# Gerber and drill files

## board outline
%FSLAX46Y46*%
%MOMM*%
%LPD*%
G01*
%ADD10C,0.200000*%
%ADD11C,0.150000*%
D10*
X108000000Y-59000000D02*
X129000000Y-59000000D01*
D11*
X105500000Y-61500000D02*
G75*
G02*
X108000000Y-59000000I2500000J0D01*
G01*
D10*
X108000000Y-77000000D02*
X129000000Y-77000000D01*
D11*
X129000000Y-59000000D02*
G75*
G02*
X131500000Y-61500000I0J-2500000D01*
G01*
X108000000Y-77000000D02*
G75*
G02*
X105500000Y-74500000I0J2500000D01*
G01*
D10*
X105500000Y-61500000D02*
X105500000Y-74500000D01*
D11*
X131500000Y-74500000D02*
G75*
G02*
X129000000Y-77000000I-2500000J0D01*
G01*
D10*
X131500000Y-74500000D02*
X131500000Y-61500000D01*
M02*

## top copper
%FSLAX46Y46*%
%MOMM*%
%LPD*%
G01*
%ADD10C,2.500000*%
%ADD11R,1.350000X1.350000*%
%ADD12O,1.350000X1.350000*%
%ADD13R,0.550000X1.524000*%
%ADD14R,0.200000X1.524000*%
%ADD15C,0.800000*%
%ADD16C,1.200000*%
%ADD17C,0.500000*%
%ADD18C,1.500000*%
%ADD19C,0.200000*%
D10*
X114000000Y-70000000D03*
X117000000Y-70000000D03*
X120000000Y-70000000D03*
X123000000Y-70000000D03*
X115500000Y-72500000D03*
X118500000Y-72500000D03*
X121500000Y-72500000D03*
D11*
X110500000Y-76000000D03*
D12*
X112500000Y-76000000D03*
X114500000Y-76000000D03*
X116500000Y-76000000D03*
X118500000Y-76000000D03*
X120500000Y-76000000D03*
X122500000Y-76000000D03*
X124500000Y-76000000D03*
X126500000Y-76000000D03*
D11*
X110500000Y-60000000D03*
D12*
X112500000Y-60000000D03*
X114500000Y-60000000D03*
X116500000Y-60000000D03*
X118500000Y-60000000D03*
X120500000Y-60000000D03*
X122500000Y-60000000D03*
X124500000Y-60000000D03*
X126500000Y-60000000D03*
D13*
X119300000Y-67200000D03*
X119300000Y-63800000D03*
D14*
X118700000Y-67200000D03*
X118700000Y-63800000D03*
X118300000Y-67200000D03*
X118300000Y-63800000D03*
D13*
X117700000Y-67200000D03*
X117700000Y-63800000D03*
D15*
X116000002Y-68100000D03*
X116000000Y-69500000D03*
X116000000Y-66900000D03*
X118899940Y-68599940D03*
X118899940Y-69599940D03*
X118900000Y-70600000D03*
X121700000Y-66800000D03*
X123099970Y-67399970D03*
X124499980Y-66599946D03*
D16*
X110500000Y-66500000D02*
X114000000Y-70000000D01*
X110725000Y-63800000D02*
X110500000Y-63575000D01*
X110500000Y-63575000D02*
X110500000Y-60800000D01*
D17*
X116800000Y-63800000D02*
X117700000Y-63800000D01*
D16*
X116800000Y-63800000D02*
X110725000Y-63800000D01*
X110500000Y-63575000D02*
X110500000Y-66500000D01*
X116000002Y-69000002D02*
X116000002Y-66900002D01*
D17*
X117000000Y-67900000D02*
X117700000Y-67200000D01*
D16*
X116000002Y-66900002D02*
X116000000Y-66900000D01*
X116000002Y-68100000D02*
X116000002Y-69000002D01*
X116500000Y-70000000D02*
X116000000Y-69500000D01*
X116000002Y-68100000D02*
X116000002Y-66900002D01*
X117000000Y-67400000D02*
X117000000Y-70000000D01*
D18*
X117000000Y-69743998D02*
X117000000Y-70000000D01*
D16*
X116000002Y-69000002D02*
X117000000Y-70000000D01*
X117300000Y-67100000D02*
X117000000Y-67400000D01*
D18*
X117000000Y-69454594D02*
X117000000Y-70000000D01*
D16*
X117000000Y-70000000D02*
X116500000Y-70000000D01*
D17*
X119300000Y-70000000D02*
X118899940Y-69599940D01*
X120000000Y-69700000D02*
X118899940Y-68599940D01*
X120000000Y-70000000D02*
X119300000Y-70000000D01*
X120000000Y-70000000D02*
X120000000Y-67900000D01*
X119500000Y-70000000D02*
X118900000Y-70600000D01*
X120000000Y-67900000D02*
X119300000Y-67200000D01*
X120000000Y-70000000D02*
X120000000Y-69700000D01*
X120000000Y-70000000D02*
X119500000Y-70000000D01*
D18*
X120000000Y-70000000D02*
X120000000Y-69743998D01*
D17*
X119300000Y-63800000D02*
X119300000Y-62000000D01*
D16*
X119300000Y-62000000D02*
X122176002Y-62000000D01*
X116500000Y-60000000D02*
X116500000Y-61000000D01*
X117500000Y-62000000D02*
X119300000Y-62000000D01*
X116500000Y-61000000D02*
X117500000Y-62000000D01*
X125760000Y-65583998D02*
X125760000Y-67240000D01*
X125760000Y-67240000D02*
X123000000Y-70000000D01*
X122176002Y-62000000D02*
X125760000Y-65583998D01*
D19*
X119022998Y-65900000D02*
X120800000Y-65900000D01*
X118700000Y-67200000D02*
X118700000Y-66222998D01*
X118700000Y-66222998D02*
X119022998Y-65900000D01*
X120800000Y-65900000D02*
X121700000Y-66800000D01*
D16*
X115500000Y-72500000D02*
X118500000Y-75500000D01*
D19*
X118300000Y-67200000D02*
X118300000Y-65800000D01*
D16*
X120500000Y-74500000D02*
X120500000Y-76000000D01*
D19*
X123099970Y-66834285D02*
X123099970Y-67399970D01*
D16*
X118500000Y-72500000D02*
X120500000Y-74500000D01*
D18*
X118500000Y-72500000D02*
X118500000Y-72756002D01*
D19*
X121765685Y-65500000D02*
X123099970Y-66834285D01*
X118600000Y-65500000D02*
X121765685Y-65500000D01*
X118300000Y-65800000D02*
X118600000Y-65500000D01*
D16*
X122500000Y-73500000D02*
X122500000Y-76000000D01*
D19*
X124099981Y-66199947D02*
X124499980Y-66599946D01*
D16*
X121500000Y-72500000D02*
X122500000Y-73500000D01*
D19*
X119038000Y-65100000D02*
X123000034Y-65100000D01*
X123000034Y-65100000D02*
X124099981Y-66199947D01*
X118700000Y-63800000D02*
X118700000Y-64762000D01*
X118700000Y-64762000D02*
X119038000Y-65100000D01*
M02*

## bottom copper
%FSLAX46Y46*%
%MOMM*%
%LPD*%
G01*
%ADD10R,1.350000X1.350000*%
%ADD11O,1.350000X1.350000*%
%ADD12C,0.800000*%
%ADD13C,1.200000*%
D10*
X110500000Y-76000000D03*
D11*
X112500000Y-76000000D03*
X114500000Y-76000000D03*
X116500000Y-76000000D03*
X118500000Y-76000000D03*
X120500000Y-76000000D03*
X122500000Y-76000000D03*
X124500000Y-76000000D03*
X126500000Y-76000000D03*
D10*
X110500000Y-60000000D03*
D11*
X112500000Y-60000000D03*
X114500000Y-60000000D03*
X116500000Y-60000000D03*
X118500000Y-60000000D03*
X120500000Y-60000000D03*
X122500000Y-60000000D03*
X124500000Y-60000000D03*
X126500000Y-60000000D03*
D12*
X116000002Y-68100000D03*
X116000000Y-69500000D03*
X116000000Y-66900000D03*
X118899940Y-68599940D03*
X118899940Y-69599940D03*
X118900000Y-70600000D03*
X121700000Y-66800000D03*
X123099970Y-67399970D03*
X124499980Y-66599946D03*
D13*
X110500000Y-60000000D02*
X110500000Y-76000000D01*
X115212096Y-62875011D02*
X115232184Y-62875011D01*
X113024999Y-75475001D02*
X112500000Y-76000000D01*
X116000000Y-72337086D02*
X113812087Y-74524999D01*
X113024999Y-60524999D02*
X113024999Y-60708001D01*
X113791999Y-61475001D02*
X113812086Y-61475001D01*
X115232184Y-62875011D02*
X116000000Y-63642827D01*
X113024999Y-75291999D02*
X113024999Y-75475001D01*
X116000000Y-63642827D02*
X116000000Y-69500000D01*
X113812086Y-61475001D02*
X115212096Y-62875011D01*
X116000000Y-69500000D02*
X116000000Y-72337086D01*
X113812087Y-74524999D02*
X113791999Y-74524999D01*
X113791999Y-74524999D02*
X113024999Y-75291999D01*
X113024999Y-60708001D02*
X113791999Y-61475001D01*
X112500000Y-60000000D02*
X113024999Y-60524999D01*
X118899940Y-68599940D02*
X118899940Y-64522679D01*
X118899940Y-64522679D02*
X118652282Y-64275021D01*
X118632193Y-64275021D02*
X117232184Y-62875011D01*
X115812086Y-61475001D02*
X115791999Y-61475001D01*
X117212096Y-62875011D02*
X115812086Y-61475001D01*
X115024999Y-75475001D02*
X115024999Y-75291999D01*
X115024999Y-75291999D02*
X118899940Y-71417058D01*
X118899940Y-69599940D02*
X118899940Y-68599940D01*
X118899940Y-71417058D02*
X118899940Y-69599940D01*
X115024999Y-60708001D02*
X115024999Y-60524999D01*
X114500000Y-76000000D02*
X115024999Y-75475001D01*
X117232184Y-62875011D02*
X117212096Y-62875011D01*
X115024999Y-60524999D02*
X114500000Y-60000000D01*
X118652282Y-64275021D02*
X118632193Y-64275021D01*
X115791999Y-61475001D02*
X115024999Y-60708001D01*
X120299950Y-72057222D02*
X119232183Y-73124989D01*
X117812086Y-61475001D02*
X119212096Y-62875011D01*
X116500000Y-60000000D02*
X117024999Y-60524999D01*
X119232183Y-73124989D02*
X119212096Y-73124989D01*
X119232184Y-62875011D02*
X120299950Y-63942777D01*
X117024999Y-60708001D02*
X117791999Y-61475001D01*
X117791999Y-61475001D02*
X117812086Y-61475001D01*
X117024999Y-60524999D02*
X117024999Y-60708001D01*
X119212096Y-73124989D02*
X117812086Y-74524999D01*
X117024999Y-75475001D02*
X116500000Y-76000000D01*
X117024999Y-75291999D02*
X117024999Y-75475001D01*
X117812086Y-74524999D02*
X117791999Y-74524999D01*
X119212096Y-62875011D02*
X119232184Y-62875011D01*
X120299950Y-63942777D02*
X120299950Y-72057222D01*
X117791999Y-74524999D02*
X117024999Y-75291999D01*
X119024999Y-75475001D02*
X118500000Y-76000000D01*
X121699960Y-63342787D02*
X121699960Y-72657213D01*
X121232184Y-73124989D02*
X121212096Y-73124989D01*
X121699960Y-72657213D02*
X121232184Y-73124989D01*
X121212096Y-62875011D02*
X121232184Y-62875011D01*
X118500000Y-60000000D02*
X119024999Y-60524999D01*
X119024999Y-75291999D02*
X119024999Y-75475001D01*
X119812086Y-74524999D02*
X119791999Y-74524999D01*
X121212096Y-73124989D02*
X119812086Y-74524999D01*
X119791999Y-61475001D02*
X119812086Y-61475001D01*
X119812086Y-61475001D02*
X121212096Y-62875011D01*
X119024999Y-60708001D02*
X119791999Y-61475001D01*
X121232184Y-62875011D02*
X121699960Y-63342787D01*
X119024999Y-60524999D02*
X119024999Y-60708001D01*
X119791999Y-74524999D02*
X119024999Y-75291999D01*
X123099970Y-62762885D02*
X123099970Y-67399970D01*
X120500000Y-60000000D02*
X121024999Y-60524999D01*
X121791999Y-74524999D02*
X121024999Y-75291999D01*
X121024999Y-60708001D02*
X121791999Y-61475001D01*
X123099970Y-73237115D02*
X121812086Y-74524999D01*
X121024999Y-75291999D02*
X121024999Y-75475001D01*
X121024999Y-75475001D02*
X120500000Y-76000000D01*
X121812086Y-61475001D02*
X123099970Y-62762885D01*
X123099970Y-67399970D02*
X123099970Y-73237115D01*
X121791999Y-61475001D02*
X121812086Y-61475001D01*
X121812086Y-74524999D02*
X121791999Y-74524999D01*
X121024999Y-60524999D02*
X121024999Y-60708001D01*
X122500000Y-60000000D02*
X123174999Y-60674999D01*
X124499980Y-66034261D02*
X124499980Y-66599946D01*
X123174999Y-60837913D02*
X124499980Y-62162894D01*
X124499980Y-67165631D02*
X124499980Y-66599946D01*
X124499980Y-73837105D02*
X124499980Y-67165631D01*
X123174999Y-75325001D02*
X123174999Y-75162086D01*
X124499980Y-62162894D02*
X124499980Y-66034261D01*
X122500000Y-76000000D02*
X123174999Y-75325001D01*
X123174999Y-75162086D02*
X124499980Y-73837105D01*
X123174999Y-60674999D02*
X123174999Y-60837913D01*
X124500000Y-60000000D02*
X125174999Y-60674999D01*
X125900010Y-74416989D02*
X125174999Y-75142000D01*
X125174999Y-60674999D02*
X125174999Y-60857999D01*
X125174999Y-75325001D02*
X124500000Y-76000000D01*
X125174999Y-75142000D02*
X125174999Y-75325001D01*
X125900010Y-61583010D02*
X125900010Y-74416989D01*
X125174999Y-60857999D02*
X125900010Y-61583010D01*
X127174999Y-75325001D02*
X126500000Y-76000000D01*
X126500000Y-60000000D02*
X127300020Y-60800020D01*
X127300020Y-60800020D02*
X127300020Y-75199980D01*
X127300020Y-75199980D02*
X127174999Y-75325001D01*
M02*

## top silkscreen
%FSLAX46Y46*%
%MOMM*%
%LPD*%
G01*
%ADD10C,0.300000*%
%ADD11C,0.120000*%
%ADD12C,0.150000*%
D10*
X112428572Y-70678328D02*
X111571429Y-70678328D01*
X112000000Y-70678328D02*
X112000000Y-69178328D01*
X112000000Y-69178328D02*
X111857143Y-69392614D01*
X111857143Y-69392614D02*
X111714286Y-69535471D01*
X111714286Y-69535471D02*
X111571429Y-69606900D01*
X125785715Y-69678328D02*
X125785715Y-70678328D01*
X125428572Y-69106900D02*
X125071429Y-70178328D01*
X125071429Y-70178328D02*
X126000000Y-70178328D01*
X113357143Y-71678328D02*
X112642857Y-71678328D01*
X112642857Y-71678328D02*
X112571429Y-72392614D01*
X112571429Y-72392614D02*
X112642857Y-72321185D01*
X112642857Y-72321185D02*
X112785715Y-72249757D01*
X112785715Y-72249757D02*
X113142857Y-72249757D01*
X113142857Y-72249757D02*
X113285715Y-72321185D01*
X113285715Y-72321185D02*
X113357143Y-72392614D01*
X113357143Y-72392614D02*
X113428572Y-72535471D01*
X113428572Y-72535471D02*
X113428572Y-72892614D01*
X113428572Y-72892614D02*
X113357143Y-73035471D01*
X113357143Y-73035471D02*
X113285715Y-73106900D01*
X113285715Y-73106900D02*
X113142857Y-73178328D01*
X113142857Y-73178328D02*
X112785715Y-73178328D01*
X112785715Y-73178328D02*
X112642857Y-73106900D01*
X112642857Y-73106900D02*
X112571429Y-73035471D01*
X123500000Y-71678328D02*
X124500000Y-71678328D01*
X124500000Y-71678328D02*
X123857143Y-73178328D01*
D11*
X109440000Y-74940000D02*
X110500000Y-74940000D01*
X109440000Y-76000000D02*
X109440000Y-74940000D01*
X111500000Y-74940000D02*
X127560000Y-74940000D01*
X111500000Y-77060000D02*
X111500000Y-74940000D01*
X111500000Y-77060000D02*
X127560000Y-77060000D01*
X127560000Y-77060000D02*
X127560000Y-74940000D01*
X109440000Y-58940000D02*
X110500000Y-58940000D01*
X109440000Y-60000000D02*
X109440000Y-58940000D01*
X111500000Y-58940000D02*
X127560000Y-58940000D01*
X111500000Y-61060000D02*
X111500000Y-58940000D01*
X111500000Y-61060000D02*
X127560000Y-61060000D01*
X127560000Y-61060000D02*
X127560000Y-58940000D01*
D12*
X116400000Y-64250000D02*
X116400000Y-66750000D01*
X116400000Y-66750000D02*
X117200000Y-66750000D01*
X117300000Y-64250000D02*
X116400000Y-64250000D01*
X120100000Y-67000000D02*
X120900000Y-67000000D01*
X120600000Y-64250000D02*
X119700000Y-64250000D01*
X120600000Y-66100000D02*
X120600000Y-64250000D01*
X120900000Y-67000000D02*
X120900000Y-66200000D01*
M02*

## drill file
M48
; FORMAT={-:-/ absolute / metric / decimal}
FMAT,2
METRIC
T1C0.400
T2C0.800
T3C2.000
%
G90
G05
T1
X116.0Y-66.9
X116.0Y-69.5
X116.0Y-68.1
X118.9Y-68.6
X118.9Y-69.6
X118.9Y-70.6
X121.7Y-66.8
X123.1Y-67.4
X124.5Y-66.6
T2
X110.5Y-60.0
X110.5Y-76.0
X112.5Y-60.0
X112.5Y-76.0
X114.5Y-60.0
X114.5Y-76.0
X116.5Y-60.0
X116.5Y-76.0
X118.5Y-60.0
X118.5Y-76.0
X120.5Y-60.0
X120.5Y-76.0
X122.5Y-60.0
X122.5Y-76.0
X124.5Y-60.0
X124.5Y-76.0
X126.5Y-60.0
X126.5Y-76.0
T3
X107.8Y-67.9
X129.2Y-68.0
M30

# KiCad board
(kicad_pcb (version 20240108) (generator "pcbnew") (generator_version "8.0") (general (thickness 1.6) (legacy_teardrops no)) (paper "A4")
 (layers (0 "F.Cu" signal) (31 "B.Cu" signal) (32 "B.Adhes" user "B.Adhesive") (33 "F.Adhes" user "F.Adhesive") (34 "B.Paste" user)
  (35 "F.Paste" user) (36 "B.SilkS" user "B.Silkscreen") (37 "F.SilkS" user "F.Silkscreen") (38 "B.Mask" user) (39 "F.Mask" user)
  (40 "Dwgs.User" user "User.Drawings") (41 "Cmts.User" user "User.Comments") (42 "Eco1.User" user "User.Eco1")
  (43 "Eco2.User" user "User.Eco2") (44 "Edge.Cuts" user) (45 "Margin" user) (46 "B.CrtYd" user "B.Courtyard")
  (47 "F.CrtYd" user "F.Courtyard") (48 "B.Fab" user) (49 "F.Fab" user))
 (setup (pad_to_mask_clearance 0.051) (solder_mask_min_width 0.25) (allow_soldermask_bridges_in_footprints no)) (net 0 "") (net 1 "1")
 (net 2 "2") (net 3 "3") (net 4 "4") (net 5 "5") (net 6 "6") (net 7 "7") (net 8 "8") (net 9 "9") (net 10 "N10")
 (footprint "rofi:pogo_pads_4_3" (layer "F.Cu") (at 118.5 70)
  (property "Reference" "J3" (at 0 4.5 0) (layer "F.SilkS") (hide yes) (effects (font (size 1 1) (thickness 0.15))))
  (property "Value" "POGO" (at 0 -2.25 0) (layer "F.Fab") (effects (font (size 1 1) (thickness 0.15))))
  (pad "1" smd circle (at -4.5 0) (size 2.5 2.5) (layers "F.Cu" "F.Paste" "F.Mask") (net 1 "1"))
  (pad "2" smd circle (at -1.5 0) (size 2.5 2.5) (layers "F.Cu" "F.Paste" "F.Mask") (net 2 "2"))
  (pad "3" smd circle (at 1.5 0) (size 2.5 2.5) (layers "F.Cu" "F.Paste" "F.Mask") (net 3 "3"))
  (pad "4" smd circle (at 4.5 0) (size 2.5 2.5) (layers "F.Cu" "F.Paste" "F.Mask") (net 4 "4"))
  (pad "5" smd circle (at -3 2.5) (size 2.5 2.5) (layers "F.Cu" "F.Paste" "F.Mask") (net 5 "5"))
  (pad "6" smd circle (at 0 2.5) (size 2.5 2.5) (layers "F.Cu" "F.Paste" "F.Mask") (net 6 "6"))
  (pad "7" smd circle (at 3 2.5) (size 2.5 2.5) (layers "F.Cu" "F.Paste" "F.Mask") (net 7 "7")))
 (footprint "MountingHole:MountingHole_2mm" (layer "F.Cu") (at 129.2 68)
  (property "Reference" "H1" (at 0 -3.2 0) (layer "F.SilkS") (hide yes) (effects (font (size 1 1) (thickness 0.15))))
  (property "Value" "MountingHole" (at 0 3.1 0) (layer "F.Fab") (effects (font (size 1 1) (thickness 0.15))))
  (pad "" np_thru_hole circle (at 0 0) (size 2 2) (drill 2) (layers "*.Cu" "*.Mask")))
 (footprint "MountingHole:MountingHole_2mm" (layer "F.Cu") (at 107.8 67.9)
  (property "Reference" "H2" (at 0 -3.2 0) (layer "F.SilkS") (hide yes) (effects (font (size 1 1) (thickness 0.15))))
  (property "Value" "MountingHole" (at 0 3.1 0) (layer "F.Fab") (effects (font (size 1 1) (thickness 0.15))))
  (pad "" np_thru_hole circle (at 0 0) (size 2 2) (drill 2) (layers "*.Cu" "*.Mask")))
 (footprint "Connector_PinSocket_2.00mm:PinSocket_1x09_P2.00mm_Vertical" (layer "F.Cu") (at 110.5 76 90)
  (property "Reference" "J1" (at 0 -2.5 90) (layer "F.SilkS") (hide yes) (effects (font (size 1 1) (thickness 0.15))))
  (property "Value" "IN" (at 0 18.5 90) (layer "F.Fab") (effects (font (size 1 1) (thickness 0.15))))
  (fp_line (start 1.06 -1.06) (end 1.06 0) (stroke (width 0.12) (type solid)) (layer "F.SilkS"))
  (fp_line (start 0 -1.06) (end 1.06 -1.06) (stroke (width 0.12) (type solid)) (layer "F.SilkS"))
  (fp_line (start 1.06 1) (end 1.06 17.06) (stroke (width 0.12) (type solid)) (layer "F.SilkS"))
  (fp_line (start -1.06 1) (end 1.06 1) (stroke (width 0.12) (type solid)) (layer "F.SilkS"))
  (fp_line (start -1.06 1) (end -1.06 17.06) (stroke (width 0.12) (type solid)) (layer "F.SilkS"))
  (fp_line (start -1.06 17.06) (end 1.06 17.06) (stroke (width 0.12) (type solid)) (layer "F.SilkS"))
  (pad "1" thru_hole rect (at 0 0 90) (size 1.35 1.35) (drill 0.8) (layers "*.Cu" "*.Mask") (remove_unused_layers no) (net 1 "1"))
  (pad "2" thru_hole oval (at 0 2 90) (size 1.35 1.35) (drill 0.8) (layers "*.Cu" "*.Mask") (remove_unused_layers no) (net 2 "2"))
  (pad "3" thru_hole oval (at 0 4 90) (size 1.35 1.35) (drill 0.8) (layers "*.Cu" "*.Mask") (remove_unused_layers no) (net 3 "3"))
  (pad "4" thru_hole oval (at 0 6 90) (size 1.35 1.35) (drill 0.8) (layers "*.Cu" "*.Mask") (remove_unused_layers no) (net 4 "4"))
  (pad "5" thru_hole oval (at 0 8 90) (size 1.35 1.35) (drill 0.8) (layers "*.Cu" "*.Mask") (remove_unused_layers no) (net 5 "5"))
  (pad "6" thru_hole oval (at 0 10 90) (size 1.35 1.35) (drill 0.8) (layers "*.Cu" "*.Mask") (remove_unused_layers no) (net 6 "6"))
  (pad "7" thru_hole oval (at 0 12 90) (size 1.35 1.35) (drill 0.8) (layers "*.Cu" "*.Mask") (remove_unused_layers no) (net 7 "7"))
  (pad "8" thru_hole oval (at 0 14 90) (size 1.35 1.35) (drill 0.8) (layers "*.Cu" "*.Mask") (remove_unused_layers no) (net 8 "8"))
  (pad "9" thru_hole oval (at 0 16 90) (size 1.35 1.35) (drill 0.8) (layers "*.Cu" "*.Mask") (remove_unused_layers no) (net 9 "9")))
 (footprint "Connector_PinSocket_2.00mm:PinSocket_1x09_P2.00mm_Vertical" (layer "F.Cu") (at 110.5 60 90)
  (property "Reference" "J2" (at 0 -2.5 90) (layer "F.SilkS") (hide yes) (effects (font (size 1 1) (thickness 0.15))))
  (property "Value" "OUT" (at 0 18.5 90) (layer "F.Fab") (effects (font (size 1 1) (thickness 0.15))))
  (fp_line (start 1.06 -1.06) (end 1.06 0) (stroke (width 0.12) (type solid)) (layer "F.SilkS"))
  (fp_line (start 0 -1.06) (end 1.06 -1.06) (stroke (width 0.12) (type solid)) (layer "F.SilkS"))
  (fp_line (start 1.06 1) (end 1.06 17.06) (stroke (width 0.12) (type solid)) (layer "F.SilkS"))
  (fp_line (start -1.06 1) (end 1.06 1) (stroke (width 0.12) (type solid)) (layer "F.SilkS"))
  (fp_line (start -1.06 1) (end -1.06 17.06) (stroke (width 0.12) (type solid)) (layer "F.SilkS"))
  (fp_line (start -1.06 17.06) (end 1.06 17.06) (stroke (width 0.12) (type solid)) (layer "F.SilkS"))
  (pad "1" thru_hole rect (at 0 0 90) (size 1.35 1.35) (drill 0.8) (layers "*.Cu" "*.Mask") (remove_unused_layers no) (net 1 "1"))
  (pad "2" thru_hole oval (at 0 2 90) (size 1.35 1.35) (drill 0.8) (layers "*.Cu" "*.Mask") (remove_unused_layers no) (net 2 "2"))
  (pad "3" thru_hole oval (at 0 4 90) (size 1.35 1.35) (drill 0.8) (layers "*.Cu" "*.Mask") (remove_unused_layers no) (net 3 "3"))
  (pad "4" thru_hole oval (at 0 6 90) (size 1.35 1.35) (drill 0.8) (layers "*.Cu" "*.Mask") (remove_unused_layers no) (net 4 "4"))
  (pad "5" thru_hole oval (at 0 8 90) (size 1.35 1.35) (drill 0.8) (layers "*.Cu" "*.Mask") (remove_unused_layers no) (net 5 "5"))
  (pad "6" thru_hole oval (at 0 10 90) (size 1.35 1.35) (drill 0.8) (layers "*.Cu" "*.Mask") (remove_unused_layers no) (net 6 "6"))
  (pad "7" thru_hole oval (at 0 12 90) (size 1.35 1.35) (drill 0.8) (layers "*.Cu" "*.Mask") (remove_unused_layers no) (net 7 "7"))
  (pad "8" thru_hole oval (at 0 14 90) (size 1.35 1.35) (drill 0.8) (layers "*.Cu" "*.Mask") (remove_unused_layers no) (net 8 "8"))
  (pad "9" thru_hole oval (at 0 16 90) (size 1.35 1.35) (drill 0.8) (layers "*.Cu" "*.Mask") (remove_unused_layers no) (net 9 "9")))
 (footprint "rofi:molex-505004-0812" (layer "F.Cu") (at 118.5 65.5 180)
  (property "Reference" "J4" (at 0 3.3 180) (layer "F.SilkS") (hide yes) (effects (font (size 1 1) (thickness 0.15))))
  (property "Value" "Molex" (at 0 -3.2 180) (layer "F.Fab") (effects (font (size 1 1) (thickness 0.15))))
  (fp_line (start 2.1 1.25) (end 2.1 -1.25) (stroke (width 0.15) (type solid)) (layer "F.SilkS"))
  (fp_line (start 2.1 -1.25) (end 1.3 -1.25) (stroke (width 0.15) (type solid)) (layer "F.SilkS"))
  (fp_line (start 1.2 1.25) (end 2.1 1.25) (stroke (width 0.15) (type solid)) (layer "F.SilkS"))
  (fp_line (start -1.6 -1.5) (end -2.4 -1.5) (stroke (width 0.15) (type solid)) (layer "F.SilkS"))
  (fp_line (start -2.1 1.25) (end -1.2 1.25) (stroke (width 0.15) (type solid)) (layer "F.SilkS"))
  (fp_line (start -2.1 -0.6) (end -2.1 1.25) (stroke (width 0.15) (type solid)) (layer "F.SilkS"))
  (fp_line (start -2.4 -1.5) (end -2.4 -0.7) (stroke (width 0.15) (type solid)) (layer "F.SilkS"))
  (pad "1" smd rect (at -0.8 -1.7 180) (size 0.55 1.524) (layers "F.Cu" "F.Paste" "F.Mask") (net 3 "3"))
  (pad "2" smd rect (at -0.8 1.7 180) (size 0.55 1.524) (layers "F.Cu" "F.Paste" "F.Mask") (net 4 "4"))
  (pad "3" smd rect (at -0.2 -1.7 180) (size 0.2 1.524) (layers "F.Cu" "F.Paste" "F.Mask") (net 5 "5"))
  (pad "4" smd rect (at -0.2 1.7 180) (size 0.2 1.524) (layers "F.Cu" "F.Paste" "F.Mask") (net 7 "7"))
  (pad "5" smd rect (at 0.2 -1.7 180) (size 0.2 1.524) (layers "F.Cu" "F.Paste" "F.Mask") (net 6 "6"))
  (pad "6" smd rect (at 0.2 1.7 180) (size 0.2 1.524) (layers "F.Cu" "F.Paste" "F.Mask") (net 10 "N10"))
  (pad "7" smd rect (at 0.8 -1.7 180) (size 0.55 1.524) (layers "F.Cu" "F.Paste" "F.Mask") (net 2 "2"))
  (pad "8" smd rect (at 0.8 1.7 180) (size 0.55 1.524) (layers "F.Cu" "F.Paste" "F.Mask") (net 1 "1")))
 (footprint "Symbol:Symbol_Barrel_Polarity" (layer "B.Cu") (at 118.7 63.5 180)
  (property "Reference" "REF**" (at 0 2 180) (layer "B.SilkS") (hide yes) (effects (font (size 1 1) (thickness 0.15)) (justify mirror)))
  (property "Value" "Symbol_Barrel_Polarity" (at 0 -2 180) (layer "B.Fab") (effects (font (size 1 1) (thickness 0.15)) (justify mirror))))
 (gr_line (start 108 59) (end 129 59) (stroke (width 0.2) (type solid)) (layer "Edge.Cuts"))
 (gr_arc (start 105.5 61.5) (mid 106.232233 59.732233) (end 108 59) (stroke (width 0.15) (type solid)) (layer "Edge.Cuts"))
 (gr_line (start 108 77) (end 129 77) (stroke (width 0.2) (type solid)) (layer "Edge.Cuts"))
 (gr_arc (start 129 59) (mid 130.767767 59.732233) (end 131.5 61.5) (stroke (width 0.15) (type solid)) (layer "Edge.Cuts"))
 (gr_arc (start 108 77) (mid 106.232233 76.267767) (end 105.5 74.5) (stroke (width 0.15) (type solid)) (layer "Edge.Cuts"))
 (gr_line (start 105.5 61.5) (end 105.5 74.5) (stroke (width 0.2) (type solid)) (layer "Edge.Cuts"))
 (gr_arc (start 131.5 74.5) (mid 130.767767 76.267767) (end 129 77) (stroke (width 0.15) (type solid)) (layer "Edge.Cuts"))
 (gr_line (start 131.5 74.5) (end 131.5 61.5) (stroke (width 0.2) (type solid)) (layer "Edge.Cuts"))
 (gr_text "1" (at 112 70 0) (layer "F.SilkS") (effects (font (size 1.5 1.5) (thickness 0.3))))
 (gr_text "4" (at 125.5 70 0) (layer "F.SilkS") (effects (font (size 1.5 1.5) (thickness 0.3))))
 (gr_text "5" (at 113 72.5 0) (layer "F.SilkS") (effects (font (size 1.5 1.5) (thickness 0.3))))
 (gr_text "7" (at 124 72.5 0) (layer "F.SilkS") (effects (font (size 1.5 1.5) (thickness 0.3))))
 (segment (start 110.5 66.5) (end 114 70) (width 1.2) (layer "F.Cu") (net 1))
 (segment (start 110.725 63.8) (end 110.5 63.575) (width 1.2) (layer "F.Cu") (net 1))
 (segment (start 110.5 63.575) (end 110.5 60.8) (width 1.2) (layer "F.Cu") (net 1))
 (segment (start 116.8 63.8) (end 117.7 63.8) (width 0.5) (layer "F.Cu") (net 1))
 (segment (start 116.8 63.8) (end 110.725 63.8) (width 1.2) (layer "F.Cu") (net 1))
 (segment (start 110.5 63.575) (end 110.5 66.5) (width 1.2) (layer "F.Cu") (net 1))
 (segment (start 110.5 60) (end 110.5 76) (width 1.2) (layer "B.Cu") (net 1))
 (segment (start 116.000002 69.000002) (end 116.000002 66.900002) (width 1.2) (layer "F.Cu") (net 2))
 (segment (start 117 67.9) (end 117.7 67.2) (width 0.5) (layer "F.Cu") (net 2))
 (segment (start 116.000002 66.900002) (end 116 66.9) (width 1.2) (layer "F.Cu") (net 2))
 (segment (start 116.000002 68.1) (end 116.000002 69.000002) (width 1.2) (layer "F.Cu") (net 2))
 (segment (start 116.5 70) (end 116 69.5) (width 1.2) (layer "F.Cu") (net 2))
 (segment (start 116.000002 68.1) (end 116.000002 66.900002) (width 1.2) (layer "F.Cu") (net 2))
 (segment (start 117 67.4) (end 117 70) (width 1.2) (layer "F.Cu") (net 2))
 (segment (start 117 69.743998) (end 117 70) (width 1.5) (layer "F.Cu") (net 2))
 (segment (start 116.000002 69.000002) (end 117 70) (width 1.2) (layer "F.Cu") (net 2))
 (segment (start 117.3 67.1) (end 117 67.4) (width 1.2) (layer "F.Cu") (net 2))
 (segment (start 117 69.454594) (end 117 70) (width 1.5) (layer "F.Cu") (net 2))
 (segment (start 117 70) (end 116.5 70) (width 1.2) (layer "F.Cu") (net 2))
 (via (at 116.000002 68.1) (size 0.8) (drill 0.4) (layers "F.Cu" "B.Cu") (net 2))
 (via (at 116 69.5) (size 0.8) (drill 0.4) (layers "F.Cu" "B.Cu") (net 2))
 (via (at 116 66.9) (size 0.8) (drill 0.4) (layers "F.Cu" "B.Cu") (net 2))
 (segment (start 115.212096 62.875011) (end 115.232184 62.875011) (width 1.2) (layer "B.Cu") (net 2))
 (segment (start 113.024999 75.475001) (end 112.5 76) (width 1.2) (layer "B.Cu") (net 2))
 (segment (start 116 72.337086) (end 113.812087 74.524999) (width 1.2) (layer "B.Cu") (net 2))
 (segment (start 113.024999 60.524999) (end 113.024999 60.708001) (width 1.2) (layer "B.Cu") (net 2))
 (segment (start 113.791999 61.475001) (end 113.812086 61.475001) (width 1.2) (layer "B.Cu") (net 2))
 (segment (start 115.232184 62.875011) (end 116 63.642827) (width 1.2) (layer "B.Cu") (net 2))
 (segment (start 113.024999 75.291999) (end 113.024999 75.475001) (width 1.2) (layer "B.Cu") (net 2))
 (segment (start 116 63.642827) (end 116 69.5) (width 1.2) (layer "B.Cu") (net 2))
 (segment (start 113.812086 61.475001) (end 115.212096 62.875011) (width 1.2) (layer "B.Cu") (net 2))
 (segment (start 116 69.5) (end 116 72.337086) (width 1.2) (layer "B.Cu") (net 2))
 (segment (start 113.812087 74.524999) (end 113.791999 74.524999) (width 1.2) (layer "B.Cu") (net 2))
 (segment (start 113.791999 74.524999) (end 113.024999 75.291999) (width 1.2) (layer "B.Cu") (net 2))
 (segment (start 113.024999 60.708001) (end 113.791999 61.475001) (width 1.2) (layer "B.Cu") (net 2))
 (segment (start 112.5 60) (end 113.024999 60.524999) (width 1.2) (layer "B.Cu") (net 2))
 (segment (start 119.3 70) (end 118.89994 69.59994) (width 0.5) (layer "F.Cu") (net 3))
 (segment (start 120 69.7) (end 118.89994 68.59994) (width 0.5) (layer "F.Cu") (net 3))
 (segment (start 120 70) (end 119.3 70) (width 0.5) (layer "F.Cu") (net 3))
 (segment (start 120 70) (end 120 67.9) (width 0.5) (layer "F.Cu") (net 3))
 (segment (start 119.5 70) (end 118.9 70.6) (width 0.5) (layer "F.Cu") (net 3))
 (segment (start 120 67.9) (end 119.3 67.2) (width 0.5) (layer "F.Cu") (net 3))
 (segment (start 120 70) (end 120 69.7) (width 0.5) (layer "F.Cu") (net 3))
 (segment (start 120 70) (end 119.5 70) (width 0.5) (layer "F.Cu") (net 3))
 (segment (start 120 70) (end 120 69.743998) (width 1.5) (layer "F.Cu") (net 3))
 (via (at 118.89994 68.59994) (size 0.8) (drill 0.4) (layers "F.Cu" "B.Cu") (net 3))
 (via (at 118.89994 69.59994) (size 0.8) (drill 0.4) (layers "F.Cu" "B.Cu") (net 3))
 (via (at 118.9 70.6) (size 0.8) (drill 0.4) (layers "F.Cu" "B.Cu") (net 3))
 (segment (start 118.89994 68.59994) (end 118.89994 64.522679) (width 1.2) (layer "B.Cu") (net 3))
 (segment (start 118.89994 64.522679) (end 118.652282 64.275021) (width 1.2) (layer "B.Cu") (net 3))
 (segment (start 118.632193 64.275021) (end 117.232184 62.875011) (width 1.2) (layer "B.Cu") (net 3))
 (segment (start 115.812086 61.475001) (end 115.791999 61.475001) (width 1.2) (layer "B.Cu") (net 3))
 (segment (start 117.212096 62.875011) (end 115.812086 61.475001) (width 1.2) (layer "B.Cu") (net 3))
 (segment (start 115.024999 75.475001) (end 115.024999 75.291999) (width 1.2) (layer "B.Cu") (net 3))
 (segment (start 115.024999 75.291999) (end 118.89994 71.417058) (width 1.2) (layer "B.Cu") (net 3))
 (segment (start 118.89994 69.59994) (end 118.89994 68.59994) (width 1.2) (layer "B.Cu") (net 3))
 (segment (start 118.89994 71.417058) (end 118.89994 69.59994) (width 1.2) (layer "B.Cu") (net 3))
 (segment (start 115.024999 60.708001) (end 115.024999 60.524999) (width 1.2) (layer "B.Cu") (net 3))
 (segment (start 114.5 76) (end 115.024999 75.475001) (width 1.2) (layer "B.Cu") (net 3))
 (segment (start 117.232184 62.875011) (end 117.212096 62.875011) (width 1.2) (layer "B.Cu") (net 3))
 (segment (start 115.024999 60.524999) (end 114.5 60) (width 1.2) (layer "B.Cu") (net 3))
 (segment (start 118.652282 64.275021) (end 118.632193 64.275021) (width 1.2) (layer "B.Cu") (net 3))
 (segment (start 115.791999 61.475001) (end 115.024999 60.708001) (width 1.2) (layer "B.Cu") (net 3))
 (segment (start 119.3 63.8) (end 119.3 62) (width 0.5) (layer "F.Cu") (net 4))
 (segment (start 119.3 62) (end 122.176002 62) (width 1.2) (layer "F.Cu") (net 4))
 (segment (start 116.5 60) (end 116.5 61) (width 1.2) (layer "F.Cu") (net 4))
 (segment (start 117.5 62) (end 119.3 62) (width 1.2) (layer "F.Cu") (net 4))
 (segment (start 116.5 61) (end 117.5 62) (width 1.2) (layer "F.Cu") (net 4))
 (segment (start 125.76 65.583998) (end 125.76 67.24) (width 1.2) (layer "F.Cu") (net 4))
 (segment (start 125.76 67.24) (end 123 70) (width 1.2) (layer "F.Cu") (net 4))
 (segment (start 122.176002 62) (end 125.76 65.583998) (width 1.2) (layer "F.Cu") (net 4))
 (segment (start 120.29995 72.057222) (end 119.232183 73.124989) (width 1.2) (layer "B.Cu") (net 4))
 (segment (start 117.812086 61.475001) (end 119.212096 62.875011) (width 1.2) (layer "B.Cu") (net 4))
 (segment (start 116.5 60) (end 117.024999 60.524999) (width 1.2) (layer "B.Cu") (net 4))
 (segment (start 119.232183 73.124989) (end 119.212096 73.124989) (width 1.2) (layer "B.Cu") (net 4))
 (segment (start 119.232184 62.875011) (end 120.29995 63.942777) (width 1.2) (layer "B.Cu") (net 4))
 (segment (start 117.024999 60.708001) (end 117.791999 61.475001) (width 1.2) (layer "B.Cu") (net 4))
 (segment (start 117.791999 61.475001) (end 117.812086 61.475001) (width 1.2) (layer "B.Cu") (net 4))
 (segment (start 117.024999 60.524999) (end 117.024999 60.708001) (width 1.2) (layer "B.Cu") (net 4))
 (segment (start 119.212096 73.124989) (end 117.812086 74.524999) (width 1.2) (layer "B.Cu") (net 4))
 (segment (start 117.024999 75.475001) (end 116.5 76) (width 1.2) (layer "B.Cu") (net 4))
 (segment (start 117.024999 75.291999) (end 117.024999 75.475001) (width 1.2) (layer "B.Cu") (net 4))
 (segment (start 117.812086 74.524999) (end 117.791999 74.524999) (width 1.2) (layer "B.Cu") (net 4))
 (segment (start 119.212096 62.875011) (end 119.232184 62.875011) (width 1.2) (layer "B.Cu") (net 4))
 (segment (start 120.29995 63.942777) (end 120.29995 72.057222) (width 1.2) (layer "B.Cu") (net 4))
 (segment (start 117.791999 74.524999) (end 117.024999 75.291999) (width 1.2) (layer "B.Cu") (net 4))
 (segment (start 119.022998 65.9) (end 120.8 65.9) (width 0.2) (layer "F.Cu") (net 5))
 (segment (start 118.7 67.2) (end 118.7 66.222998) (width 0.2) (layer "F.Cu") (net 5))
 (segment (start 118.7 66.222998) (end 119.022998 65.9) (width 0.2) (layer "F.Cu") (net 5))
 (segment (start 120.8 65.9) (end 121.7 66.8) (width 0.2) (layer "F.Cu") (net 5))
 (segment (start 115.5 72.5) (end 118.5 75.5) (width 1.2) (layer "F.Cu") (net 5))
 (via (at 121.7 66.8) (size 0.8) (drill 0.4) (layers "F.Cu" "B.Cu") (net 5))
 (segment (start 119.024999 75.475001) (end 118.5 76) (width 1.2) (layer "B.Cu") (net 5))
 (segment (start 121.69996 63.342787) (end 121.69996 72.657213) (width 1.2) (layer "B.Cu") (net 5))
 (segment (start 121.232184 73.124989) (end 121.212096 73.124989) (width 1.2) (layer "B.Cu") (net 5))
 (segment (start 121.69996 72.657213) (end 121.232184 73.124989) (width 1.2) (layer "B.Cu") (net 5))
 (segment (start 121.212096 62.875011) (end 121.232184 62.875011) (width 1.2) (layer "B.Cu") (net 5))
 (segment (start 118.5 60) (end 119.024999 60.524999) (width 1.2) (layer "B.Cu") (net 5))
 (segment (start 119.024999 75.291999) (end 119.024999 75.475001) (width 1.2) (layer "B.Cu") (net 5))
 (segment (start 119.812086 74.524999) (end 119.791999 74.524999) (width 1.2) (layer "B.Cu") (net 5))
 (segment (start 121.212096 73.124989) (end 119.812086 74.524999) (width 1.2) (layer "B.Cu") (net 5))
 (segment (start 119.791999 61.475001) (end 119.812086 61.475001) (width 1.2) (layer "B.Cu") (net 5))
 (segment (start 119.812086 61.475001) (end 121.212096 62.875011) (width 1.2) (layer "B.Cu") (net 5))
 (segment (start 119.024999 60.708001) (end 119.791999 61.475001) (width 1.2) (layer "B.Cu") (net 5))
 (segment (start 121.232184 62.875011) (end 121.69996 63.342787) (width 1.2) (layer "B.Cu") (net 5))
 (segment (start 119.024999 60.524999) (end 119.024999 60.708001) (width 1.2) (layer "B.Cu") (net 5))
 (segment (start 119.791999 74.524999) (end 119.024999 75.291999) (width 1.2) (layer "B.Cu") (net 5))
 (segment (start 118.3 67.2) (end 118.3 65.8) (width 0.2) (layer "F.Cu") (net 6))
 (segment (start 120.5 74.5) (end 120.5 76) (width 1.2) (layer "F.Cu") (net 6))
 (segment (start 123.09997 66.834285) (end 123.09997 67.39997) (width 0.2) (layer "F.Cu") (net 6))
 (segment (start 118.5 72.5) (end 120.5 74.5) (width 1.2) (layer "F.Cu") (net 6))
 (segment (start 118.5 72.5) (end 118.5 72.756002) (width 1.5) (layer "F.Cu") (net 6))
 (segment (start 121.765685 65.5) (end 123.09997 66.834285) (width 0.2) (layer "F.Cu") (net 6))
 (segment (start 118.6 65.5) (end 121.765685 65.5) (width 0.2) (layer "F.Cu") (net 6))
 (segment (start 118.3 65.8) (end 118.6 65.5) (width 0.2) (layer "F.Cu") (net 6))
 (via (at 123.09997 67.39997) (size 0.8) (drill 0.4) (layers "F.Cu" "B.Cu") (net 6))
 (segment (start 123.09997 62.762885) (end 123.09997 67.39997) (width 1.2) (layer "B.Cu") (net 6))
 (segment (start 120.5 60) (end 121.024999 60.524999) (width 1.2) (layer "B.Cu") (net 6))
 (segment (start 121.791999 74.524999) (end 121.024999 75.291999) (width 1.2) (layer "B.Cu") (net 6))
 (segment (start 121.024999 60.708001) (end 121.791999 61.475001) (width 1.2) (layer "B.Cu") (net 6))
 (segment (start 123.09997 73.237115) (end 121.812086 74.524999) (width 1.2) (layer "B.Cu") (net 6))
 (segment (start 121.024999 75.291999) (end 121.024999 75.475001) (width 1.2) (layer "B.Cu") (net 6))
 (segment (start 121.024999 75.475001) (end 120.5 76) (width 1.2) (layer "B.Cu") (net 6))
 (segment (start 121.812086 61.475001) (end 123.09997 62.762885) (width 1.2) (layer "B.Cu") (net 6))
 (segment (start 123.09997 67.39997) (end 123.09997 73.237115) (width 1.2) (layer "B.Cu") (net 6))
 (segment (start 121.791999 61.475001) (end 121.812086 61.475001) (width 1.2) (layer "B.Cu") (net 6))
 (segment (start 121.812086 74.524999) (end 121.791999 74.524999) (width 1.2) (layer "B.Cu") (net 6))
 (segment (start 121.024999 60.524999) (end 121.024999 60.708001) (width 1.2) (layer "B.Cu") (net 6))
 (segment (start 122.5 73.5) (end 122.5 76) (width 1.2) (layer "F.Cu") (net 7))
 (segment (start 124.099981 66.199947) (end 124.49998 66.599946) (width 0.2) (layer "F.Cu") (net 7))
 (segment (start 121.5 72.5) (end 122.5 73.5) (width 1.2) (layer "F.Cu") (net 7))
 (segment (start 119.038 65.1) (end 123.000034 65.1) (width 0.2) (layer "F.Cu") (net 7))
 (segment (start 123.000034 65.1) (end 124.099981 66.199947) (width 0.2) (layer "F.Cu") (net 7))
 (segment (start 118.7 63.8) (end 118.7 64.762) (width 0.2) (layer "F.Cu") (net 7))
 (segment (start 118.7 64.762) (end 119.038 65.1) (width 0.2) (layer "F.Cu") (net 7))
 (via (at 124.49998 66.599946) (size 0.8) (drill 0.4) (layers "F.Cu" "B.Cu") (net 7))
 (segment (start 122.5 60) (end 123.174999 60.674999) (width 1.2) (layer "B.Cu") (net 7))
 (segment (start 124.49998 66.034261) (end 124.49998 66.599946) (width 1.2) (layer "B.Cu") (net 7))
 (segment (start 123.174999 60.837913) (end 124.49998 62.162894) (width 1.2) (layer "B.Cu") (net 7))
 (segment (start 124.49998 67.165631) (end 124.49998 66.599946) (width 1.2) (layer "B.Cu") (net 7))
 (segment (start 124.49998 73.837105) (end 124.49998 67.165631) (width 1.2) (layer "B.Cu") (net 7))
 (segment (start 123.174999 75.325001) (end 123.174999 75.162086) (width 1.2) (layer "B.Cu") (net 7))
 (segment (start 124.49998 62.162894) (end 124.49998 66.034261) (width 1.2) (layer "B.Cu") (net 7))
 (segment (start 122.5 76) (end 123.174999 75.325001) (width 1.2) (layer "B.Cu") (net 7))
 (segment (start 123.174999 75.162086) (end 124.49998 73.837105) (width 1.2) (layer "B.Cu") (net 7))
 (segment (start 123.174999 60.674999) (end 123.174999 60.837913) (width 1.2) (layer "B.Cu") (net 7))
 (segment (start 124.5 60) (end 125.174999 60.674999) (width 1.2) (layer "B.Cu") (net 8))
 (segment (start 125.90001 74.416989) (end 125.174999 75.142) (width 1.2) (layer "B.Cu") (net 8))
 (segment (start 125.174999 60.674999) (end 125.174999 60.857999) (width 1.2) (layer "B.Cu") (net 8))
 (segment (start 125.174999 75.325001) (end 124.5 76) (width 1.2) (layer "B.Cu") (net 8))
 (segment (start 125.174999 75.142) (end 125.174999 75.325001) (width 1.2) (layer "B.Cu") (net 8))
 (segment (start 125.90001 61.58301) (end 125.90001 74.416989) (width 1.2) (layer "B.Cu") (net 8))
 (segment (start 125.174999 60.857999) (end 125.90001 61.58301) (width 1.2) (layer "B.Cu") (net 8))
 (segment (start 127.174999 75.325001) (end 126.5 76) (width 1.2) (layer "B.Cu") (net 9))
 (segment (start 126.5 60) (end 127.30002 60.80002) (width 1.2) (layer "B.Cu") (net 9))
 (segment (start 127.30002 60.80002) (end 127.30002 75.19998) (width 1.2) (layer "B.Cu") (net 9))
 (segment (start 127.30002 75.19998) (end 127.174999 75.325001) (width 1.2) (layer "B.Cu") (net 9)))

